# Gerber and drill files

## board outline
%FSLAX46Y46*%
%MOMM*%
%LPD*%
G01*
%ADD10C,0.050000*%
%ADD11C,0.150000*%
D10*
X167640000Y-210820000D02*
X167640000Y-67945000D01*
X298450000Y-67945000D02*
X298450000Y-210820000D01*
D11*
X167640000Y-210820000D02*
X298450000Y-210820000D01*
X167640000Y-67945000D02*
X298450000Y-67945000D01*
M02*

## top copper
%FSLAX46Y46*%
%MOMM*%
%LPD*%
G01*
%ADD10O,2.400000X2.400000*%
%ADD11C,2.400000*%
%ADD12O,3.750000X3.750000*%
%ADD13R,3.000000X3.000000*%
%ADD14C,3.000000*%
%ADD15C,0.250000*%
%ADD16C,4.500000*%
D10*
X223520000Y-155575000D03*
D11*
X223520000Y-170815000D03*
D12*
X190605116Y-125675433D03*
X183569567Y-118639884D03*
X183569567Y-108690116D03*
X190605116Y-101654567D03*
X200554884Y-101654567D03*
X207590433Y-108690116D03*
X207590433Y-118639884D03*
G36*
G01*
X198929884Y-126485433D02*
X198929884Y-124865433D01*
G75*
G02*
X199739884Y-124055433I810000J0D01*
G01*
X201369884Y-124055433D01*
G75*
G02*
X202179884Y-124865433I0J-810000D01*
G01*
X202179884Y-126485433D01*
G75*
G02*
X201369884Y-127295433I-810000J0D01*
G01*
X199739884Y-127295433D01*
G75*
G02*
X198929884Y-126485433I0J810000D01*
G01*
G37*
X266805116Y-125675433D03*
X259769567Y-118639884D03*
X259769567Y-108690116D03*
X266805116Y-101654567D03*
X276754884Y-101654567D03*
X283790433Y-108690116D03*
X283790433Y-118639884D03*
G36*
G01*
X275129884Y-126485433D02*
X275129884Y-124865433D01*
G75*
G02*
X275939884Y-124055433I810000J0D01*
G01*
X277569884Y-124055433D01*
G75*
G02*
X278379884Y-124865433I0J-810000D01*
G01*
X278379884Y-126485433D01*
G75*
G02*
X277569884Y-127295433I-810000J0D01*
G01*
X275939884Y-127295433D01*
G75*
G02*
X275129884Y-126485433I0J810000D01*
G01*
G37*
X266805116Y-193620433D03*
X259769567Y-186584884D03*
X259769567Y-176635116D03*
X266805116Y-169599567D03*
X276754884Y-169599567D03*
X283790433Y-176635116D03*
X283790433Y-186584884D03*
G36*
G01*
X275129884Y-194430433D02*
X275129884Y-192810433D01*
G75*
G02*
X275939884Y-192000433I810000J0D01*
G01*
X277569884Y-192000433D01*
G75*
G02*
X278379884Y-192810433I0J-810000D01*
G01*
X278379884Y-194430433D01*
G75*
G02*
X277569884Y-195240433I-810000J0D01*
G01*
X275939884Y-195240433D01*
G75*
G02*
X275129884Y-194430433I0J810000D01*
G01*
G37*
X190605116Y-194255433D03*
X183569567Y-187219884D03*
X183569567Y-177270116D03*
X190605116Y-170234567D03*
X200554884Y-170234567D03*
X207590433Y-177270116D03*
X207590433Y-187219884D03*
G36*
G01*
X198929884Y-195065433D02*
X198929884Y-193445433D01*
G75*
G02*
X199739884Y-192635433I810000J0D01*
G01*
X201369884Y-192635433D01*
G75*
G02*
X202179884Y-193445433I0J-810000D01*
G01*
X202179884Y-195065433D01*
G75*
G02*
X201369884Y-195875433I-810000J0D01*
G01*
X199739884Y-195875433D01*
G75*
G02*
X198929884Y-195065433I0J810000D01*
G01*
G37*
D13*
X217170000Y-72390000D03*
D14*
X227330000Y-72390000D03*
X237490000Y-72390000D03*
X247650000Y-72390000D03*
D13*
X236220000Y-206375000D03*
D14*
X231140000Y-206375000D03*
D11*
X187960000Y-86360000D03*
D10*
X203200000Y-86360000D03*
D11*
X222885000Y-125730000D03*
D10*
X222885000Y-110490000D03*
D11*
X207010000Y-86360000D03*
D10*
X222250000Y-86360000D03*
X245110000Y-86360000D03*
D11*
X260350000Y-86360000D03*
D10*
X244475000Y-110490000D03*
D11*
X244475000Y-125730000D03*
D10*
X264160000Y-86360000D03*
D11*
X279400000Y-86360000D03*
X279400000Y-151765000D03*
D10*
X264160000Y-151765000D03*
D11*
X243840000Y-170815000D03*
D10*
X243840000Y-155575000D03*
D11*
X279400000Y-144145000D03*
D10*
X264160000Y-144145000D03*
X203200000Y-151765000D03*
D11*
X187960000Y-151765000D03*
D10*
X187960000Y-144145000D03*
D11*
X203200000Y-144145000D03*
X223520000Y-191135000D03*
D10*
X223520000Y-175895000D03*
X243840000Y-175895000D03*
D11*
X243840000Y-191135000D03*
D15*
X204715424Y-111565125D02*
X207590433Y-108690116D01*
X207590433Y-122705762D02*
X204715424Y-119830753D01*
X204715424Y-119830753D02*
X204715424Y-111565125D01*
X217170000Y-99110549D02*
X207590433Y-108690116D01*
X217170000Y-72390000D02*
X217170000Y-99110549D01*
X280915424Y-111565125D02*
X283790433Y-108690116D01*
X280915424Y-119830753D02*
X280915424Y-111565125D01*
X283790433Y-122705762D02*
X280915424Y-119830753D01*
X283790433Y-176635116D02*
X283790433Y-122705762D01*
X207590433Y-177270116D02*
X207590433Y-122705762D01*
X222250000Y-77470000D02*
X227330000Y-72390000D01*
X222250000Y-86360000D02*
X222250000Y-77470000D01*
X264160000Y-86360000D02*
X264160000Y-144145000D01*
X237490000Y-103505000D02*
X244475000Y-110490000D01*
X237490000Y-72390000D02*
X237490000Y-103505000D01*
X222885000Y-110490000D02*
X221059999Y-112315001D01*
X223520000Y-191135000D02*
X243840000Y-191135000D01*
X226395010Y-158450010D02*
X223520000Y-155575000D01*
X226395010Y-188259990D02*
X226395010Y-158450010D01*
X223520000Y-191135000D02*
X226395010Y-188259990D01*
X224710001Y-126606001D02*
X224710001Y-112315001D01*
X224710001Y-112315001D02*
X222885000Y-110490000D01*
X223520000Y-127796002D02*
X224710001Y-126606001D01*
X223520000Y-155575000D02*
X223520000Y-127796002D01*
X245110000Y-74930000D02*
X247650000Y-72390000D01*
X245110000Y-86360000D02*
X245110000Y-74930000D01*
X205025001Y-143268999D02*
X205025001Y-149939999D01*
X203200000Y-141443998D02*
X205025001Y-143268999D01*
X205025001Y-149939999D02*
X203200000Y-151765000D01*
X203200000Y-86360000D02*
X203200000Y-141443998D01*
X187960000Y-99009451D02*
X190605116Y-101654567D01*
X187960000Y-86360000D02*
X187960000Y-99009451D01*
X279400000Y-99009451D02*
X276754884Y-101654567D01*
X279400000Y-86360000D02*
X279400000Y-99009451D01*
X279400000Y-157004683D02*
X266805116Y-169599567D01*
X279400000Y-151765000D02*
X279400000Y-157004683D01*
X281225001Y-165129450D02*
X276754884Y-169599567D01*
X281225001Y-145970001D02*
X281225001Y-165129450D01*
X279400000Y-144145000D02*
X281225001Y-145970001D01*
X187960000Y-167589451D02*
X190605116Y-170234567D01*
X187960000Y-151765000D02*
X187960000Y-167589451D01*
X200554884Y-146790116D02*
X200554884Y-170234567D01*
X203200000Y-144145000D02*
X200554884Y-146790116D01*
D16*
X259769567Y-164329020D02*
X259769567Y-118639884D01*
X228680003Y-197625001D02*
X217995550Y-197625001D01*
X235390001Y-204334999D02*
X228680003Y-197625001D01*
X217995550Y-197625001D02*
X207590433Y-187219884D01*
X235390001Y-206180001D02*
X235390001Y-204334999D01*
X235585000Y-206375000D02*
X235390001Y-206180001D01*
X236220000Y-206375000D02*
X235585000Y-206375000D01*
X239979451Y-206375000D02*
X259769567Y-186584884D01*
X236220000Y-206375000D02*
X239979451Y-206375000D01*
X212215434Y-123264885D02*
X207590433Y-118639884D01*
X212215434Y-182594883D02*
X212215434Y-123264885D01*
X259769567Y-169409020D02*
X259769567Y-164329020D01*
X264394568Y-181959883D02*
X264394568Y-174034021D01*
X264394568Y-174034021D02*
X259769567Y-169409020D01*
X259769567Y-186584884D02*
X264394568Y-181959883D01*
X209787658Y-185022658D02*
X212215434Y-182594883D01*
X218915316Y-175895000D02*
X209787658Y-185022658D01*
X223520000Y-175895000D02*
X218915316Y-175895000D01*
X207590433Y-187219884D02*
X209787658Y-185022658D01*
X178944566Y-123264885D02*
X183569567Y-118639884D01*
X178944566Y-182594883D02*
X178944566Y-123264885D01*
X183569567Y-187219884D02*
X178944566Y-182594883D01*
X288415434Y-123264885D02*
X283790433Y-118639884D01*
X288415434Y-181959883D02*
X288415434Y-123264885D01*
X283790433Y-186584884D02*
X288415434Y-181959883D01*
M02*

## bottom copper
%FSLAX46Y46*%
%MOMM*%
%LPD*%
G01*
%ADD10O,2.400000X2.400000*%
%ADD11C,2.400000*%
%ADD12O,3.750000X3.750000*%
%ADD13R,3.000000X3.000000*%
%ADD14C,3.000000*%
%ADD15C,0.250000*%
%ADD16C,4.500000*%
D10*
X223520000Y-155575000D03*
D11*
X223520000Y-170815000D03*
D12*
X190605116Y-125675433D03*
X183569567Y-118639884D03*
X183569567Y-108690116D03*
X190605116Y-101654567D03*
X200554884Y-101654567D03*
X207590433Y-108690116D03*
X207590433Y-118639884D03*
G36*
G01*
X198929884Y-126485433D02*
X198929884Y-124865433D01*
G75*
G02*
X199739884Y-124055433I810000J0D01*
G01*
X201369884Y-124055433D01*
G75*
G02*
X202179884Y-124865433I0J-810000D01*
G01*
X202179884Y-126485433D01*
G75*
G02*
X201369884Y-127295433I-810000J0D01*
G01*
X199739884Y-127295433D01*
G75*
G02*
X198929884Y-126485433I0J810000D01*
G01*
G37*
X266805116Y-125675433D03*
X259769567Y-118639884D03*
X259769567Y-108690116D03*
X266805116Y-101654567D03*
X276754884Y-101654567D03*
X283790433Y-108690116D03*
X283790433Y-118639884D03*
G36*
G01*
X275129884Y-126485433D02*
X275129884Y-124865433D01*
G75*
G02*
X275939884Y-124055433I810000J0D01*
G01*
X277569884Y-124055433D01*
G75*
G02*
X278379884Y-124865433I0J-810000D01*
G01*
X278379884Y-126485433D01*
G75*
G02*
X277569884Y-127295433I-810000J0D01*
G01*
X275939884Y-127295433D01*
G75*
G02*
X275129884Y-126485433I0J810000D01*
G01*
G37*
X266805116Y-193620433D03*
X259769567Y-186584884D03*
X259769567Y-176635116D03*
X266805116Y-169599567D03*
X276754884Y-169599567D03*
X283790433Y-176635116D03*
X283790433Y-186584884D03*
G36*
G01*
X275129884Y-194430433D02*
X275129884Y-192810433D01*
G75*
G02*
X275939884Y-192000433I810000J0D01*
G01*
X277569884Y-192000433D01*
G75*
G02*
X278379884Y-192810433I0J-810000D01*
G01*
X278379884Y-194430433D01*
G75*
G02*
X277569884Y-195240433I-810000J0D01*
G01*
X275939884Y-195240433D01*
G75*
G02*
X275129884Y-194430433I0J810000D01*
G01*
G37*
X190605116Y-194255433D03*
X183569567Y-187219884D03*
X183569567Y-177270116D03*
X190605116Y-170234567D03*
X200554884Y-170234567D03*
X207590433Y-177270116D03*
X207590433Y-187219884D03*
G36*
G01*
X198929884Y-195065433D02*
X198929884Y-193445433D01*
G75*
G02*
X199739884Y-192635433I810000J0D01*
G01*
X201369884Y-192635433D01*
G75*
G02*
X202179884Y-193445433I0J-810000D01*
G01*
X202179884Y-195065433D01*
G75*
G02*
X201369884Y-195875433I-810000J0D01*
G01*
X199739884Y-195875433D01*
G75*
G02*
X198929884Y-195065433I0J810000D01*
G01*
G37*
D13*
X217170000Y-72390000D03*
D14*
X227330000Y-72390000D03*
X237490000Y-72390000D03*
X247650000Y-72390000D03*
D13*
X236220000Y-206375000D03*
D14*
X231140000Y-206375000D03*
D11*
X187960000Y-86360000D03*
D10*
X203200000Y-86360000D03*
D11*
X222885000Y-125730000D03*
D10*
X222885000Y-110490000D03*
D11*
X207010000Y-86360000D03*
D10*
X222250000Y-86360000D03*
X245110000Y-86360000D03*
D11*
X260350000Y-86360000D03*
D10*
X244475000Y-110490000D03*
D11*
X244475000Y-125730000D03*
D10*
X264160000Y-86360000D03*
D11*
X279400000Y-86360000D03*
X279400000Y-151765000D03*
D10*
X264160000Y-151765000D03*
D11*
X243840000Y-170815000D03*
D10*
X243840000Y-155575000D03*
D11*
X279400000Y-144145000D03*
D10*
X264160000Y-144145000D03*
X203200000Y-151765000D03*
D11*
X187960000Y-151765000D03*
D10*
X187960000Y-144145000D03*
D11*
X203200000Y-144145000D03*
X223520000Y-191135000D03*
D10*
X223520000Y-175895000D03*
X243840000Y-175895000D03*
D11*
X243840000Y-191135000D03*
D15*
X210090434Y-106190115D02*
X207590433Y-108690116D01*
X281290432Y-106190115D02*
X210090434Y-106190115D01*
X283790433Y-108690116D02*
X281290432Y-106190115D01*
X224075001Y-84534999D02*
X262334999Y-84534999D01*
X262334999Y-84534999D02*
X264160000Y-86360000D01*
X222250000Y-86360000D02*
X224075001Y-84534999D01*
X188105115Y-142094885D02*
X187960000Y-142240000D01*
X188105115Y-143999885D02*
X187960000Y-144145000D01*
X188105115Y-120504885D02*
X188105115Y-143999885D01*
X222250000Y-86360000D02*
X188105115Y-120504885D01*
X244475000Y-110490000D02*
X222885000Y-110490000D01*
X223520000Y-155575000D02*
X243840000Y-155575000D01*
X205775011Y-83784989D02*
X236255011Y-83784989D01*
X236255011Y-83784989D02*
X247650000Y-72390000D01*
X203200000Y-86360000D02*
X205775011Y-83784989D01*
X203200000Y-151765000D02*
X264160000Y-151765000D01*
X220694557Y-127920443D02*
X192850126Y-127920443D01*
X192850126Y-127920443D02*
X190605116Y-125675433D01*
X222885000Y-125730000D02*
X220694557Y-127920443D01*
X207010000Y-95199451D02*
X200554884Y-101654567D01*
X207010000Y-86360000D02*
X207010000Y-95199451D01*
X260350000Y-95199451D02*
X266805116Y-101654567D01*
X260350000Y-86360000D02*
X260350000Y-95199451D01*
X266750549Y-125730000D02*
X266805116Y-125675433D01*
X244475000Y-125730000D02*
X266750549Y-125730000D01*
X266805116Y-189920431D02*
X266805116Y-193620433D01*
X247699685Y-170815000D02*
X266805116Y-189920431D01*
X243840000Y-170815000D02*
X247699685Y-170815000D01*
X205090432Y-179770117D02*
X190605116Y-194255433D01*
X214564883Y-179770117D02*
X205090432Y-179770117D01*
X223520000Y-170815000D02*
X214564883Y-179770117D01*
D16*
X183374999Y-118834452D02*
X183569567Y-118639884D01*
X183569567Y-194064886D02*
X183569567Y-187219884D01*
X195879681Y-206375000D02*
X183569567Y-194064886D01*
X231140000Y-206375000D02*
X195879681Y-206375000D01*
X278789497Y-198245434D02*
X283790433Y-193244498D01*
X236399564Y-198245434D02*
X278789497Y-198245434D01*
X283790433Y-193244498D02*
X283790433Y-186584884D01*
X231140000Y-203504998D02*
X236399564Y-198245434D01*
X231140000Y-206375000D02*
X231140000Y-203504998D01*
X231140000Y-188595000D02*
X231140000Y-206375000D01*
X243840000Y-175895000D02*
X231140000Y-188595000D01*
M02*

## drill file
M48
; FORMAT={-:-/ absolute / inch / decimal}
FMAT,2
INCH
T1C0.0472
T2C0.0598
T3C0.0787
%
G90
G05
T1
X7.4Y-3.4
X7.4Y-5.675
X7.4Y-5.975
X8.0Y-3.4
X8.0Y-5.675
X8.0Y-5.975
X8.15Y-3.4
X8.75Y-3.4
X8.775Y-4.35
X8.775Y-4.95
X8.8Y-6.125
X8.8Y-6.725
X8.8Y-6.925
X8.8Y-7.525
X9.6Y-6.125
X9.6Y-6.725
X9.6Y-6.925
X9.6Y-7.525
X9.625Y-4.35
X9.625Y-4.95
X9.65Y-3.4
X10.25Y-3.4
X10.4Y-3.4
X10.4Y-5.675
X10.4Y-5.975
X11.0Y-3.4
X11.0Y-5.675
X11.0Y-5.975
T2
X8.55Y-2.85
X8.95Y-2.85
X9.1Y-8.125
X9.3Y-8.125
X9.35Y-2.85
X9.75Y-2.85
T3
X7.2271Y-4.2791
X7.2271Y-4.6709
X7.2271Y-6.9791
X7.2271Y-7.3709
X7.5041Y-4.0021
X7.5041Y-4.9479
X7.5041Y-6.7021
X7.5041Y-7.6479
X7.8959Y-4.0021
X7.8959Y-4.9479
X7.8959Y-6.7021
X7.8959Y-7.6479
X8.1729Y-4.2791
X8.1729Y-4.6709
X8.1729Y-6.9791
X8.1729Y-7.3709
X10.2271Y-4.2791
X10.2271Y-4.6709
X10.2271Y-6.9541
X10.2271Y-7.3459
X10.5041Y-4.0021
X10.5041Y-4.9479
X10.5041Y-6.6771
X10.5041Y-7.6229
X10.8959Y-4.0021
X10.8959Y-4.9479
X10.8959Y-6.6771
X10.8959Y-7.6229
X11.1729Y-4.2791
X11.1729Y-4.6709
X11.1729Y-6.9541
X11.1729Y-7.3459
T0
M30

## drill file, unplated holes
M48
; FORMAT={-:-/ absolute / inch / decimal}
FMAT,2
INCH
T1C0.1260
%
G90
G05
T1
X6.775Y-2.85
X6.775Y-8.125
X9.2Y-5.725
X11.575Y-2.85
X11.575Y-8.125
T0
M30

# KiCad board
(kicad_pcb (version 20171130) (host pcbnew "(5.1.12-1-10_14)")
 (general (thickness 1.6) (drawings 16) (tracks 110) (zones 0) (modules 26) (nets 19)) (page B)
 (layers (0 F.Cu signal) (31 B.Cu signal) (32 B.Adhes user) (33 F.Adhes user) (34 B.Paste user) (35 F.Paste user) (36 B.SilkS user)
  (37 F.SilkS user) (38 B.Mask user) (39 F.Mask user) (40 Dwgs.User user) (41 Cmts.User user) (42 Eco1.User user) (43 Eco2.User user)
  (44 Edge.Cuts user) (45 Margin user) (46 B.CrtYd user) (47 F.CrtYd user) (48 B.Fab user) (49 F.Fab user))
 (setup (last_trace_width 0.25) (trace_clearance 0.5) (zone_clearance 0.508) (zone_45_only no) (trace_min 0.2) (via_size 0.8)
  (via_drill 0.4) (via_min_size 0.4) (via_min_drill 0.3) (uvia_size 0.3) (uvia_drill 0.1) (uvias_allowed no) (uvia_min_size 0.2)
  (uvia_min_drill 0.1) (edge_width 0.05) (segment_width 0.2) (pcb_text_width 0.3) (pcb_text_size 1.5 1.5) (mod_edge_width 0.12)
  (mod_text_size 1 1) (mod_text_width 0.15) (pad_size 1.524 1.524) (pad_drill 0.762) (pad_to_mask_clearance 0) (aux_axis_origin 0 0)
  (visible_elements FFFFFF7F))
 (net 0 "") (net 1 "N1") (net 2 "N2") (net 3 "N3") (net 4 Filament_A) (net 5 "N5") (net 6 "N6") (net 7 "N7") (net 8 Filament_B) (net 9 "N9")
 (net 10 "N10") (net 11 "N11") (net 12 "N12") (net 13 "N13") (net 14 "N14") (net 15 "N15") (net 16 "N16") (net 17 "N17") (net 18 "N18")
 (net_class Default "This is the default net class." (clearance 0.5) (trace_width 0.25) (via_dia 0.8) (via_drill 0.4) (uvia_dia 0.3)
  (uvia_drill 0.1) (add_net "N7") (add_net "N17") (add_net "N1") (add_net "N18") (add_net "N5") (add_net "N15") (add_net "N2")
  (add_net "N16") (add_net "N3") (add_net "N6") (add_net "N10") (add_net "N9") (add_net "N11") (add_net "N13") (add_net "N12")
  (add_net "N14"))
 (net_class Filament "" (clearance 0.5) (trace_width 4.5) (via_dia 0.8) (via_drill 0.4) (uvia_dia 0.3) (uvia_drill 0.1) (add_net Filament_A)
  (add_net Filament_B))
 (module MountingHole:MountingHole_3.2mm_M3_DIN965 (layer F.Cu) (at 294.005 206.375)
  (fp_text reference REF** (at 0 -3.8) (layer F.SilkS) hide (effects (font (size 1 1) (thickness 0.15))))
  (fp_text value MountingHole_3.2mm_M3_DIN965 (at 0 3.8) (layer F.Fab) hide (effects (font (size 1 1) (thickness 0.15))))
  (pad 1 np_thru_hole circle (at 0 0) (size 3.2 3.2) (drill 3.2) (layers *.Cu *.Mask)))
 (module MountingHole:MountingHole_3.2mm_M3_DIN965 (layer F.Cu) (at 172.085 206.375)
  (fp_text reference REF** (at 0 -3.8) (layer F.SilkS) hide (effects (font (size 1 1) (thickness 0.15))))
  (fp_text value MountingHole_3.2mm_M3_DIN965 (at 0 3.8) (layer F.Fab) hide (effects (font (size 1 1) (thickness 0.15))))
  (pad 1 np_thru_hole circle (at 0 0) (size 3.2 3.2) (drill 3.2) (layers *.Cu *.Mask)))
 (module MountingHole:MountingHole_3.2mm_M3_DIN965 (layer F.Cu) (at 172.085 72.39)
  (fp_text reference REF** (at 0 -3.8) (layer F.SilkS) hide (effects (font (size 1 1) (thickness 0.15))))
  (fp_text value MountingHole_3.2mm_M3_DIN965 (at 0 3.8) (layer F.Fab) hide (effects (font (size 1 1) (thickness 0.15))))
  (pad 1 np_thru_hole circle (at 0 0) (size 3.2 3.2) (drill 3.2) (layers *.Cu *.Mask)))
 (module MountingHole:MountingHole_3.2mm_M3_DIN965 (layer F.Cu) (at 294.005 72.39)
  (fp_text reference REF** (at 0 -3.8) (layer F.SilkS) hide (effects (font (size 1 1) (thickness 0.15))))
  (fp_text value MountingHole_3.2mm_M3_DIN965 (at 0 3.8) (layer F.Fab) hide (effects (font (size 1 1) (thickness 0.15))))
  (pad 1 np_thru_hole circle (at 0 0) (size 3.2 3.2) (drill 3.2) (layers *.Cu *.Mask)))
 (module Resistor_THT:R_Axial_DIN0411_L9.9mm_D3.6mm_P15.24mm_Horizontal (layer F.Cu) (at 223.52 170.815 90)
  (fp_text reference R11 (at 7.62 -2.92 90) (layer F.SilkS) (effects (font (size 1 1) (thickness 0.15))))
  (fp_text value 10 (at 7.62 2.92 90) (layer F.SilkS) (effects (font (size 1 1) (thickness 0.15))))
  (pad 2 thru_hole oval (at 15.24 0 90) (size 2.4 2.4) (drill 1.2) (layers *.Cu *.Mask) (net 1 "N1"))
  (pad 1 thru_hole circle (at 0 0 90) (size 2.4 2.4) (drill 1.2) (layers *.Cu *.Mask) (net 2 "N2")))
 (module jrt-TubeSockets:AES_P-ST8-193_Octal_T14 (layer F.Cu) (at 195.58 113.665)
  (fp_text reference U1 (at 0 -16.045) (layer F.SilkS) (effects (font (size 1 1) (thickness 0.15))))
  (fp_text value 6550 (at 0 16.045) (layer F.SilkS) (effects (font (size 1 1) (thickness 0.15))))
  (pad 8 thru_hole oval (at -4.974884 12.010433) (size 3.75 3.75) (drill 2) (layers *.Cu *.Mask) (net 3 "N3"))
  (pad 7 thru_hole oval (at -12.010433 4.974884) (size 3.75 3.75) (drill 2) (layers *.Cu *.Mask) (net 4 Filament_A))
  (pad 6 thru_hole oval (at -12.010433 -4.974884) (size 3.75 3.75) (drill 2) (layers *.Cu *.Mask))
  (pad 5 thru_hole oval (at -4.974884 -12.010433) (size 3.75 3.75) (drill 2) (layers *.Cu *.Mask) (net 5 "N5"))
  (pad 4 thru_hole oval (at 4.974884 -12.010433) (size 3.75 3.75) (drill 2) (layers *.Cu *.Mask) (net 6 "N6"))
  (pad 3 thru_hole oval (at 12.010433 -4.974884) (size 3.75 3.75) (drill 2) (layers *.Cu *.Mask) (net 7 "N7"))
  (pad 2 thru_hole oval (at 12.010433 4.974884) (size 3.75 3.75) (drill 2) (layers *.Cu *.Mask) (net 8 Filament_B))
  (pad 1 thru_hole roundrect (at 4.974884 12.010433) (size 3.25 3.24) (drill 2) (layers *.Cu *.Mask) (roundrect_rratio 0.25)))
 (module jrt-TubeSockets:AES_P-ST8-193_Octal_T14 (layer F.Cu) (at 271.78 113.665)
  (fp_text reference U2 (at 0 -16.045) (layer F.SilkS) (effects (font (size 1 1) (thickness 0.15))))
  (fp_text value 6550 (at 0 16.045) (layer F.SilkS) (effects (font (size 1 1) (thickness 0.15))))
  (pad 8 thru_hole oval (at -4.974884 12.010433) (size 3.75 3.75) (drill 2) (layers *.Cu *.Mask) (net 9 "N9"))
  (pad 7 thru_hole oval (at -12.010433 4.974884) (size 3.75 3.75) (drill 2) (layers *.Cu *.Mask) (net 8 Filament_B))
  (pad 6 thru_hole oval (at -12.010433 -4.974884) (size 3.75 3.75) (drill 2) (layers *.Cu *.Mask))
  (pad 5 thru_hole oval (at -4.974884 -12.010433) (size 3.75 3.75) (drill 2) (layers *.Cu *.Mask) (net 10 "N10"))
  (pad 4 thru_hole oval (at 4.974884 -12.010433) (size 3.75 3.75) (drill 2) (layers *.Cu *.Mask) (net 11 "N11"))
  (pad 3 thru_hole oval (at 12.010433 -4.974884) (size 3.75 3.75) (drill 2) (layers *.Cu *.Mask) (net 7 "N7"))
  (pad 2 thru_hole oval (at 12.010433 4.974884) (size 3.75 3.75) (drill 2) (layers *.Cu *.Mask) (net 4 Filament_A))
  (pad 1 thru_hole roundrect (at 4.974884 12.010433) (size 3.25 3.24) (drill 2) (layers *.Cu *.Mask) (roundrect_rratio 0.25)))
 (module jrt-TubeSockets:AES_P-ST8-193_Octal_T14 (layer F.Cu) (at 271.78 181.61)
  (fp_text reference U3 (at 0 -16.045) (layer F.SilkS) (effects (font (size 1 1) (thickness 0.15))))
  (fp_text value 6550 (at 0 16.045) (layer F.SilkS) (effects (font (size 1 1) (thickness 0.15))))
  (pad 8 thru_hole oval (at -4.974884 12.010433) (size 3.75 3.75) (drill 2) (layers *.Cu *.Mask) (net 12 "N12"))
  (pad 7 thru_hole oval (at -12.010433 4.974884) (size 3.75 3.75) (drill 2) (layers *.Cu *.Mask) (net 8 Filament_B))
  (pad 6 thru_hole oval (at -12.010433 -4.974884) (size 3.75 3.75) (drill 2) (layers *.Cu *.Mask))
  (pad 5 thru_hole oval (at -4.974884 -12.010433) (size 3.75 3.75) (drill 2) (layers *.Cu *.Mask) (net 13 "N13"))
  (pad 4 thru_hole oval (at 4.974884 -12.010433) (size 3.75 3.75) (drill 2) (layers *.Cu *.Mask) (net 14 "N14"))
  (pad 3 thru_hole oval (at 12.010433 -4.974884) (size 3.75 3.75) (drill 2) (layers *.Cu *.Mask) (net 7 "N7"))
  (pad 2 thru_hole oval (at 12.010433 4.974884) (size 3.75 3.75) (drill 2) (layers *.Cu *.Mask) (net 4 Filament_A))
  (pad 1 thru_hole roundrect (at 4.974884 12.010433) (size 3.25 3.24) (drill 2) (layers *.Cu *.Mask) (roundrect_rratio 0.25)))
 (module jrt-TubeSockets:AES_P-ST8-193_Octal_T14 (layer F.Cu) (at 195.58 182.245)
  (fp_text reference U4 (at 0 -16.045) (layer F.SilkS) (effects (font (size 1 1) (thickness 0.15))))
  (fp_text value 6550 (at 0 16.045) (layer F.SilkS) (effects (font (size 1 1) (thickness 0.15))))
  (pad 8 thru_hole oval (at -4.974884 12.010433) (size 3.75 3.75) (drill 2) (layers *.Cu *.Mask) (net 2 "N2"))
  (pad 7 thru_hole oval (at -12.010433 4.974884) (size 3.75 3.75) (drill 2) (layers *.Cu *.Mask) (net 4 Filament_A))
  (pad 6 thru_hole oval (at -12.010433 -4.974884) (size 3.75 3.75) (drill 2) (layers *.Cu *.Mask))
  (pad 5 thru_hole oval (at -4.974884 -12.010433) (size 3.75 3.75) (drill 2) (layers *.Cu *.Mask) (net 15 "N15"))
  (pad 4 thru_hole oval (at 4.974884 -12.010433) (size 3.75 3.75) (drill 2) (layers *.Cu *.Mask) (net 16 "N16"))
  (pad 3 thru_hole oval (at 12.010433 -4.974884) (size 3.75 3.75) (drill 2) (layers *.Cu *.Mask) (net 7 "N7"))
  (pad 2 thru_hole oval (at 12.010433 4.974884) (size 3.75 3.75) (drill 2) (layers *.Cu *.Mask) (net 8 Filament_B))
  (pad 1 thru_hole roundrect (at 4.974884 12.010433) (size 3.25 3.24) (drill 2) (layers *.Cu *.Mask) (roundrect_rratio 0.25)))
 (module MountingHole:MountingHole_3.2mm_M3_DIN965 (layer F.Cu) (at 233.68 145.415)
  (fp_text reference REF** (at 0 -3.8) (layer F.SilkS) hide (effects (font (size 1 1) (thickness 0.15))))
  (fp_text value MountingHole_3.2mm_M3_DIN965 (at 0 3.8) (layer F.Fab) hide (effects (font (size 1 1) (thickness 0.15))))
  (pad 1 np_thru_hole circle (at 0 0) (size 3.2 3.2) (drill 3.2) (layers *.Cu *.Mask)))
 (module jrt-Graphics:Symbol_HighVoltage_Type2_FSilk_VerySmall (layer F.Cu) (at 233.68 123.825)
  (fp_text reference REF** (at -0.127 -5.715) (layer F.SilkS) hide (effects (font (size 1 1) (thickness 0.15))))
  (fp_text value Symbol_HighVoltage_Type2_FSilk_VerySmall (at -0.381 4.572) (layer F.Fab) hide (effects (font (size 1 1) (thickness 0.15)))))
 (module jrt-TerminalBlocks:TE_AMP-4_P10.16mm (layer F.Cu) (at 232.41 72.39)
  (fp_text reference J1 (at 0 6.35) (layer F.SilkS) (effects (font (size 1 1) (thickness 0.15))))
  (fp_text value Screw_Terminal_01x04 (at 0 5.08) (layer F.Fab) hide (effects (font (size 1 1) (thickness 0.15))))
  (pad 1 thru_hole rect (at -15.24 0) (size 3 3) (drill 1.52) (layers *.Cu *.Mask) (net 7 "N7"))
  (pad 2 thru_hole circle (at -5.08 0) (size 3 3) (drill 1.52) (layers *.Cu *.Mask) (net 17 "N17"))
  (pad 3 thru_hole circle (at 5.08 0) (size 3 3) (drill 1.52) (layers *.Cu *.Mask) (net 1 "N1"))
  (pad 4 thru_hole circle (at 15.24 0) (size 3 3) (drill 1.52) (layers *.Cu *.Mask) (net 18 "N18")))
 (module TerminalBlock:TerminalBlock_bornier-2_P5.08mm (layer F.Cu) (at 236.22 206.375 180)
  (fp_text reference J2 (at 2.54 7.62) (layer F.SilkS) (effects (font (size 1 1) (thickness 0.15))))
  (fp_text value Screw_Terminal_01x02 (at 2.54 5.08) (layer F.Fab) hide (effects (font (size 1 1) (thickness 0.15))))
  (pad 1 thru_hole rect (at 0 0 180) (size 3 3) (drill 1.52) (layers *.Cu *.Mask) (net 8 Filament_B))
  (pad 2 thru_hole circle (at 5.08 0 180) (size 3 3) (drill 1.52) (layers *.Cu *.Mask) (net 4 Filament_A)))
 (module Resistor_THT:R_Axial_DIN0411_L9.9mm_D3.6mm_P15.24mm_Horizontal (layer F.Cu) (at 187.96 86.36)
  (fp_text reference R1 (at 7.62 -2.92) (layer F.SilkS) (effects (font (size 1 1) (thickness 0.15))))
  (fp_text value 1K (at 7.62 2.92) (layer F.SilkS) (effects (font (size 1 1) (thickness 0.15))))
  (pad 1 thru_hole circle (at 0 0) (size 2.4 2.4) (drill 1.2) (layers *.Cu *.Mask) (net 5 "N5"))
  (pad 2 thru_hole oval (at 15.24 0) (size 2.4 2.4) (drill 1.2) (layers *.Cu *.Mask) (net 18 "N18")))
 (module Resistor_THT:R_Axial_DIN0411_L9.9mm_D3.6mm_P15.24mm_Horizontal (layer F.Cu) (at 222.885 125.73 90)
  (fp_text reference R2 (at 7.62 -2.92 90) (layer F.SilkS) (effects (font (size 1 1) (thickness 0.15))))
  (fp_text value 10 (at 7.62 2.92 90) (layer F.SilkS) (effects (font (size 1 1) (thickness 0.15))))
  (pad 1 thru_hole circle (at 0 0 90) (size 2.4 2.4) (drill 1.2) (layers *.Cu *.Mask) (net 3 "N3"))
  (pad 2 thru_hole oval (at 15.24 0 90) (size 2.4 2.4) (drill 1.2) (layers *.Cu *.Mask) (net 1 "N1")))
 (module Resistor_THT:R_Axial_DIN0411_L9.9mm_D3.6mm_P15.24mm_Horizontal (layer F.Cu) (at 207.01 86.36)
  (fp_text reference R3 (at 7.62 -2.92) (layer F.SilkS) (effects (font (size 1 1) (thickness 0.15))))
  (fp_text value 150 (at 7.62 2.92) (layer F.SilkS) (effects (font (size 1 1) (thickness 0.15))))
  (pad 1 thru_hole circle (at 0 0) (size 2.4 2.4) (drill 1.2) (layers *.Cu *.Mask) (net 6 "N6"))
  (pad 2 thru_hole oval (at 15.24 0) (size 2.4 2.4) (drill 1.2) (layers *.Cu *.Mask) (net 17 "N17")))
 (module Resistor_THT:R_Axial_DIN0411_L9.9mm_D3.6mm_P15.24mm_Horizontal (layer F.Cu) (at 260.35 86.36 180)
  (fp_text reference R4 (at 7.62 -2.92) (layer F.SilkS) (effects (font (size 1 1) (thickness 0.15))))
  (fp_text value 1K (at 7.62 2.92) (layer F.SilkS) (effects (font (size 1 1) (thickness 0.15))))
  (pad 2 thru_hole oval (at 15.24 0 180) (size 2.4 2.4) (drill 1.2) (layers *.Cu *.Mask) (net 18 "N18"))
  (pad 1 thru_hole circle (at 0 0 180) (size 2.4 2.4) (drill 1.2) (layers *.Cu *.Mask) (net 10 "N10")))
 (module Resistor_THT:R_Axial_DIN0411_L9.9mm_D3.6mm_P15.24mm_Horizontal (layer F.Cu) (at 244.475 125.73 90)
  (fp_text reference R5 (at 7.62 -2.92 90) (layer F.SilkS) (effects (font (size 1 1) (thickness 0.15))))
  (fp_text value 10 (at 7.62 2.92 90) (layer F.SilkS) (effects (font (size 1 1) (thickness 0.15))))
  (pad 2 thru_hole oval (at 15.24 0 90) (size 2.4 2.4) (drill 1.2) (layers *.Cu *.Mask) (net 1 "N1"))
  (pad 1 thru_hole circle (at 0 0 90) (size 2.4 2.4) (drill 1.2) (layers *.Cu *.Mask) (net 9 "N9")))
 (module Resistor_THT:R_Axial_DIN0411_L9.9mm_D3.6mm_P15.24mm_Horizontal (layer F.Cu) (at 279.4 86.36 180)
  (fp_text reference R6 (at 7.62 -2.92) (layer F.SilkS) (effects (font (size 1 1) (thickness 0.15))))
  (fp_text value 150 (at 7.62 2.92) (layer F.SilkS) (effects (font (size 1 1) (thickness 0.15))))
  (pad 2 thru_hole oval (at 15.24 0 180) (size 2.4 2.4) (drill 1.2) (layers *.Cu *.Mask) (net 17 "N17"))
  (pad 1 thru_hole circle (at 0 0 180) (size 2.4 2.4) (drill 1.2) (layers *.Cu *.Mask) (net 11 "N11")))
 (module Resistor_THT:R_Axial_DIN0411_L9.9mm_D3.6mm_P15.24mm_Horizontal (layer F.Cu) (at 279.4 151.765 180)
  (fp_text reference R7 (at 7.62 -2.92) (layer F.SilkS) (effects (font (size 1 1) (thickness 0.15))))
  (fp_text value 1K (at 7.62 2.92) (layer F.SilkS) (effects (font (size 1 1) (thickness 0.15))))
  (pad 1 thru_hole circle (at 0 0 180) (size 2.4 2.4) (drill 1.2) (layers *.Cu *.Mask) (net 13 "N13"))
  (pad 2 thru_hole oval (at 15.24 0 180) (size 2.4 2.4) (drill 1.2) (layers *.Cu *.Mask) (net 18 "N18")))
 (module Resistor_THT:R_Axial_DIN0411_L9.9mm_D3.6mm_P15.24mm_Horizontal (layer F.Cu) (at 243.84 170.815 90)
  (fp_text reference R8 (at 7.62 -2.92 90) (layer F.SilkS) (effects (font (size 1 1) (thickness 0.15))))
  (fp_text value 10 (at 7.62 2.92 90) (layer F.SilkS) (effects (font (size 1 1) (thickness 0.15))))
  (pad 1 thru_hole circle (at 0 0 90) (size 2.4 2.4) (drill 1.2) (layers *.Cu *.Mask) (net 12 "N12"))
  (pad 2 thru_hole oval (at 15.24 0 90) (size 2.4 2.4) (drill 1.2) (layers *.Cu *.Mask) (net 1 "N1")))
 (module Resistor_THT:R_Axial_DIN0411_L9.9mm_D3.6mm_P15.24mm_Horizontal (layer F.Cu) (at 279.4 144.145 180)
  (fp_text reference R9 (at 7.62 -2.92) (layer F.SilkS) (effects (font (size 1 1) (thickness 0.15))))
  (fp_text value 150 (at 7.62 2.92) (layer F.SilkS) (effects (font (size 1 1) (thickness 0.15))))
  (pad 1 thru_hole circle (at 0 0 180) (size 2.4 2.4) (drill 1.2) (layers *.Cu *.Mask) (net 14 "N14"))
  (pad 2 thru_hole oval (at 15.24 0 180) (size 2.4 2.4) (drill 1.2) (layers *.Cu *.Mask) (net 17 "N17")))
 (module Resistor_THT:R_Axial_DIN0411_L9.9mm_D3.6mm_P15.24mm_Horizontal (layer F.Cu) (at 187.96 151.765)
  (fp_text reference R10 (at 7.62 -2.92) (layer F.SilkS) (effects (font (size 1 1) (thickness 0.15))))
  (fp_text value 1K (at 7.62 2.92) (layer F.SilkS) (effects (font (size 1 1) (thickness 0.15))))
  (pad 2 thru_hole oval (at 15.24 0) (size 2.4 2.4) (drill 1.2) (layers *.Cu *.Mask) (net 18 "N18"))
  (pad 1 thru_hole circle (at 0 0) (size 2.4 2.4) (drill 1.2) (layers *.Cu *.Mask) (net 15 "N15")))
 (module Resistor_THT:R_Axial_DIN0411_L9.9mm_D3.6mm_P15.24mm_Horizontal (layer F.Cu) (at 203.2 144.145 180)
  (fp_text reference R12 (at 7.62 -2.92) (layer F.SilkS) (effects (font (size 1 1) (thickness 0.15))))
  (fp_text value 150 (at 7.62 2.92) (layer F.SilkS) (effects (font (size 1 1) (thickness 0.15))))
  (pad 2 thru_hole oval (at 15.24 0 180) (size 2.4 2.4) (drill 1.2) (layers *.Cu *.Mask) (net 17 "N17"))
  (pad 1 thru_hole circle (at 0 0 180) (size 2.4 2.4) (drill 1.2) (layers *.Cu *.Mask) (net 16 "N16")))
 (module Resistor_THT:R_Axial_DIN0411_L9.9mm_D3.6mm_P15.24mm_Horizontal (layer F.Cu) (at 223.52 191.135 90)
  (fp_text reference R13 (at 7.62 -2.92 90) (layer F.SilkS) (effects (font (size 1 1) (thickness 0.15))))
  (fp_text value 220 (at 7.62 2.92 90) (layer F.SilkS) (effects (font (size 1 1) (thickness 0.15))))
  (pad 1 thru_hole circle (at 0 0 90) (size 2.4 2.4) (drill 1.2) (layers *.Cu *.Mask) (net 1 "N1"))
  (pad 2 thru_hole oval (at 15.24 0 90) (size 2.4 2.4) (drill 1.2) (layers *.Cu *.Mask) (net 8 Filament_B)))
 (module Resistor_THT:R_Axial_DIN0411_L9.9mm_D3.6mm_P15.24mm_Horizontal (layer F.Cu) (at 243.84 191.135 90)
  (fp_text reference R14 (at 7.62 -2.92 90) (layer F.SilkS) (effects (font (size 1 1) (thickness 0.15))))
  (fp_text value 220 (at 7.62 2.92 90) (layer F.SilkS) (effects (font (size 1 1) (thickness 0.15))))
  (pad 2 thru_hole oval (at 15.24 0 90) (size 2.4 2.4) (drill 1.2) (layers *.Cu *.Mask) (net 4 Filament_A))
  (pad 1 thru_hole circle (at 0 0 90) (size 2.4 2.4) (drill 1.2) (layers *.Cu *.Mask) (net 1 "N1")))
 (gr_line (start 167.64 210.82) (end 167.64 67.945) (layer Edge.Cuts) (width 0.05))
 (gr_line (start 298.45 67.945) (end 298.45 210.82) (layer Edge.Cuts) (width 0.05))
 (gr_line (start 167.64 210.82) (end 298.45 210.82) (layer Edge.Cuts) (width 0.15))
 (gr_line (start 167.64 67.945) (end 298.45 67.945) (layer Edge.Cuts) (width 0.15))
 (segment (start 204.715424 111.565125) (end 207.590433 108.690116) (width 0.25) (layer F.Cu) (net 7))
 (segment (start 207.590433 122.705762) (end 204.715424 119.830753) (width 0.25) (layer F.Cu) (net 7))
 (segment (start 204.715424 119.830753) (end 204.715424 111.565125) (width 0.25) (layer F.Cu) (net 7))
 (segment (start 217.17 99.110549) (end 207.590433 108.690116) (width 0.25) (layer F.Cu) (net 7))
 (segment (start 217.17 72.39) (end 217.17 99.110549) (width 0.25) (layer F.Cu) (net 7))
 (segment (start 210.090434 106.190115) (end 207.590433 108.690116) (width 0.25) (layer B.Cu) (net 7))
 (segment (start 281.290432 106.190115) (end 210.090434 106.190115) (width 0.25) (layer B.Cu) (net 7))
 (segment (start 283.790433 108.690116) (end 281.290432 106.190115) (width 0.25) (layer B.Cu) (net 7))
 (segment (start 280.915424 111.565125) (end 283.790433 108.690116) (width 0.25) (layer F.Cu) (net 7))
 (segment (start 280.915424 119.830753) (end 280.915424 111.565125) (width 0.25) (layer F.Cu) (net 7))
 (segment (start 283.790433 122.705762) (end 280.915424 119.830753) (width 0.25) (layer F.Cu) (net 7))
 (segment (start 283.790433 176.635116) (end 283.790433 122.705762) (width 0.25) (layer F.Cu) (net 7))
 (segment (start 207.590433 177.270116) (end 207.590433 122.705762) (width 0.25) (layer F.Cu) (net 7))
 (segment (start 224.075001 84.534999) (end 262.334999 84.534999) (width 0.25) (layer B.Cu) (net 17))
 (segment (start 262.334999 84.534999) (end 264.16 86.36) (width 0.25) (layer B.Cu) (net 17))
 (segment (start 222.25 86.36) (end 224.075001 84.534999) (width 0.25) (layer B.Cu) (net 17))
 (segment (start 222.25 77.47) (end 227.33 72.39) (width 0.25) (layer F.Cu) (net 17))
 (segment (start 222.25 86.36) (end 222.25 77.47) (width 0.25) (layer F.Cu) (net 17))
 (segment (start 188.105115 142.094885) (end 187.96 142.24) (width 0.25) (layer B.Cu) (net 17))
 (segment (start 188.105115 143.999885) (end 187.96 144.145) (width 0.25) (layer B.Cu) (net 17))
 (segment (start 188.105115 120.504885) (end 188.105115 143.999885) (width 0.25) (layer B.Cu) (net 17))
 (segment (start 222.25 86.36) (end 188.105115 120.504885) (width 0.25) (layer B.Cu) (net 17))
 (segment (start 264.16 86.36) (end 264.16 144.145) (width 0.25) (layer F.Cu) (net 17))
 (segment (start 237.49 103.505) (end 244.475 110.49) (width 0.25) (layer F.Cu) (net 1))
 (segment (start 237.49 72.39) (end 237.49 103.505) (width 0.25) (layer F.Cu) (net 1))
 (segment (start 244.475 110.49) (end 222.885 110.49) (width 0.25) (layer B.Cu) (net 1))
 (segment (start 222.885 110.49) (end 221.059999 112.315001) (width 0.25) (layer F.Cu) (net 1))
 (segment (start 223.52 155.575) (end 243.84 155.575) (width 0.25) (layer B.Cu) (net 1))
 (segment (start 223.52 191.135) (end 243.84 191.135) (width 0.25) (layer F.Cu) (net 1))
 (segment (start 226.39501 158.45001) (end 223.52 155.575) (width 0.25) (layer F.Cu) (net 1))
 (segment (start 226.39501 188.25999) (end 226.39501 158.45001) (width 0.25) (layer F.Cu) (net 1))
 (segment (start 223.52 191.135) (end 226.39501 188.25999) (width 0.25) (layer F.Cu) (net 1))
 (segment (start 224.710001 126.606001) (end 224.710001 112.315001) (width 0.25) (layer F.Cu) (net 1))
 (segment (start 224.710001 112.315001) (end 222.885 110.49) (width 0.25) (layer F.Cu) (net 1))
 (segment (start 223.52 127.796002) (end 224.710001 126.606001) (width 0.25) (layer F.Cu) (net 1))
 (segment (start 223.52 155.575) (end 223.52 127.796002) (width 0.25) (layer F.Cu) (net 1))
 (segment (start 245.11 74.93) (end 247.65 72.39) (width 0.25) (layer F.Cu) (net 18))
 (segment (start 245.11 86.36) (end 245.11 74.93) (width 0.25) (layer F.Cu) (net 18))
 (segment (start 205.775011 83.784989) (end 236.255011 83.784989) (width 0.25) (layer B.Cu) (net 18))
 (segment (start 236.255011 83.784989) (end 247.65 72.39) (width 0.25) (layer B.Cu) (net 18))
 (segment (start 203.2 86.36) (end 205.775011 83.784989) (width 0.25) (layer B.Cu) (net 18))
 (segment (start 203.2 151.765) (end 264.16 151.765) (width 0.25) (layer B.Cu) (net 18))
 (segment (start 205.025001 143.268999) (end 205.025001 149.939999) (width 0.25) (layer F.Cu) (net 18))
 (segment (start 203.2 141.443998) (end 205.025001 143.268999) (width 0.25) (layer F.Cu) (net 18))
 (segment (start 205.025001 149.939999) (end 203.2 151.765) (width 0.25) (layer F.Cu) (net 18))
 (segment (start 203.2 86.36) (end 203.2 141.443998) (width 0.25) (layer F.Cu) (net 18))
 (segment (start 187.96 99.009451) (end 190.605116 101.654567) (width 0.25) (layer F.Cu) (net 5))
 (segment (start 187.96 86.36) (end 187.96 99.009451) (width 0.25) (layer F.Cu) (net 5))
 (segment (start 220.694557 127.920443) (end 192.850126 127.920443) (width 0.25) (layer B.Cu) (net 3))
 (segment (start 192.850126 127.920443) (end 190.605116 125.675433) (width 0.25) (layer B.Cu) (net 3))
 (segment (start 222.885 125.73) (end 220.694557 127.920443) (width 0.25) (layer B.Cu) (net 3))
 (segment (start 207.01 95.199451) (end 200.554884 101.654567) (width 0.25) (layer B.Cu) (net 6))
 (segment (start 207.01 86.36) (end 207.01 95.199451) (width 0.25) (layer B.Cu) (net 6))
 (segment (start 260.35 95.199451) (end 266.805116 101.654567) (width 0.25) (layer B.Cu) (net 10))
 (segment (start 260.35 86.36) (end 260.35 95.199451) (width 0.25) (layer B.Cu) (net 10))
 (segment (start 266.750549 125.73) (end 266.805116 125.675433) (width 0.25) (layer B.Cu) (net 9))
 (segment (start 244.475 125.73) (end 266.750549 125.73) (width 0.25) (layer B.Cu) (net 9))
 (segment (start 279.4 99.009451) (end 276.754884 101.654567) (width 0.25) (layer F.Cu) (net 11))
 (segment (start 279.4 86.36) (end 279.4 99.009451) (width 0.25) (layer F.Cu) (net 11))
 (segment (start 279.4 157.004683) (end 266.805116 169.599567) (width 0.25) (layer F.Cu) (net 13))
 (segment (start 279.4 151.765) (end 279.4 157.004683) (width 0.25) (layer F.Cu) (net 13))
 (segment (start 266.805116 189.920431) (end 266.805116 193.620433) (width 0.25) (layer B.Cu) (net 12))
 (segment (start 247.699685 170.815) (end 266.805116 189.920431) (width 0.25) (layer B.Cu) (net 12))
 (segment (start 243.84 170.815) (end 247.699685 170.815) (width 0.25) (layer B.Cu) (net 12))
 (segment (start 281.225001 165.12945) (end 276.754884 169.599567) (width 0.25) (layer F.Cu) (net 14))
 (segment (start 281.225001 145.970001) (end 281.225001 165.12945) (width 0.25) (layer F.Cu) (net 14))
 (segment (start 279.4 144.145) (end 281.225001 145.970001) (width 0.25) (layer F.Cu) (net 14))
 (segment (start 187.96 167.589451) (end 190.605116 170.234567) (width 0.25) (layer F.Cu) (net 15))
 (segment (start 187.96 151.765) (end 187.96 167.589451) (width 0.25) (layer F.Cu) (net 15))
 (segment (start 205.090432 179.770117) (end 190.605116 194.255433) (width 0.25) (layer B.Cu) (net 2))
 (segment (start 214.564883 179.770117) (end 205.090432 179.770117) (width 0.25) (layer B.Cu) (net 2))
 (segment (start 223.52 170.815) (end 214.564883 179.770117) (width 0.25) (layer B.Cu) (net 2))
 (segment (start 200.554884 146.790116) (end 200.554884 170.234567) (width 0.25) (layer F.Cu) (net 16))
 (segment (start 203.2 144.145) (end 200.554884 146.790116) (width 0.25) (layer F.Cu) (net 16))
 (segment (start 259.769567 164.32902) (end 259.769567 118.639884) (width 4.5) (layer F.Cu) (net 8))
 (segment (start 228.680003 197.625001) (end 217.99555 197.625001) (width 4.5) (layer F.Cu) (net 8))
 (segment (start 235.390001 204.334999) (end 228.680003 197.625001) (width 4.5) (layer F.Cu) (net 8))
 (segment (start 217.99555 197.625001) (end 207.590433 187.219884) (width 4.5) (layer F.Cu) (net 8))
 (segment (start 235.390001 206.180001) (end 235.390001 204.334999) (width 4.5) (layer F.Cu) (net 8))
 (segment (start 235.585 206.375) (end 235.390001 206.180001) (width 4.5) (layer F.Cu) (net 8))
 (segment (start 236.22 206.375) (end 235.585 206.375) (width 4.5) (layer F.Cu) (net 8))
 (segment (start 239.979451 206.375) (end 259.769567 186.584884) (width 4.5) (layer F.Cu) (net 8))
 (segment (start 236.22 206.375) (end 239.979451 206.375) (width 4.5) (layer F.Cu) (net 8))
 (segment (start 212.215434 123.264885) (end 207.590433 118.639884) (width 4.5) (layer F.Cu) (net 8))
 (segment (start 212.215434 182.594883) (end 212.215434 123.264885) (width 4.5) (layer F.Cu) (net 8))
 (segment (start 259.769567 169.40902) (end 259.769567 164.32902) (width 4.5) (layer F.Cu) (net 8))
 (segment (start 264.394568 181.959883) (end 264.394568 174.034021) (width 4.5) (layer F.Cu) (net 8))
 (segment (start 264.394568 174.034021) (end 259.769567 169.40902) (width 4.5) (layer F.Cu) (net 8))
 (segment (start 259.769567 186.584884) (end 264.394568 181.959883) (width 4.5) (layer F.Cu) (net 8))
 (segment (start 209.787658 185.022658) (end 212.215434 182.594883) (width 4.5) (layer F.Cu) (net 8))
 (segment (start 218.915316 175.895) (end 209.787658 185.022658) (width 4.5) (layer F.Cu) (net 8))
 (segment (start 223.52 175.895) (end 218.915316 175.895) (width 4.5) (layer F.Cu) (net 8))
 (segment (start 207.590433 187.219884) (end 209.787658 185.022658) (width 4.5) (layer F.Cu) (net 8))
 (segment (start 183.374999 118.834452) (end 183.569567 118.639884) (width 4.5) (layer B.Cu) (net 4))
 (segment (start 183.569567 194.064886) (end 183.569567 187.219884) (width 4.5) (layer B.Cu) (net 4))
 (segment (start 195.879681 206.375) (end 183.569567 194.064886) (width 4.5) (layer B.Cu) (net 4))
 (segment (start 231.14 206.375) (end 195.879681 206.375) (width 4.5) (layer B.Cu) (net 4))
 (segment (start 278.789497 198.245434) (end 283.790433 193.244498) (width 4.5) (layer B.Cu) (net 4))
 (segment (start 236.399564 198.245434) (end 278.789497 198.245434) (width 4.5) (layer B.Cu) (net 4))
 (segment (start 283.790433 193.244498) (end 283.790433 186.584884) (width 4.5) (layer B.Cu) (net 4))
 (segment (start 231.14 203.504998) (end 236.399564 198.245434) (width 4.5) (layer B.Cu) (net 4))
 (segment (start 231.14 206.375) (end 231.14 203.504998) (width 4.5) (layer B.Cu) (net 4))
 (segment (start 231.14 188.595) (end 231.14 206.375) (width 4.5) (layer B.Cu) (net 4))
 (segment (start 243.84 175.895) (end 231.14 188.595) (width 4.5) (layer B.Cu) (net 4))
 (segment (start 178.944566 123.264885) (end 183.569567 118.639884) (width 4.5) (layer F.Cu) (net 4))
 (segment (start 178.944566 182.594883) (end 178.944566 123.264885) (width 4.5) (layer F.Cu) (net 4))
 (segment (start 183.569567 187.219884) (end 178.944566 182.594883) (width 4.5) (layer F.Cu) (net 4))
 (segment (start 288.415434 123.264885) (end 283.790433 118.639884) (width 4.5) (layer F.Cu) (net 4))
 (segment (start 288.415434 181.959883) (end 288.415434 123.264885) (width 4.5) (layer F.Cu) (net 4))
 (segment (start 283.790433 186.584884) (end 288.415434 181.959883) (width 4.5) (layer F.Cu) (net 4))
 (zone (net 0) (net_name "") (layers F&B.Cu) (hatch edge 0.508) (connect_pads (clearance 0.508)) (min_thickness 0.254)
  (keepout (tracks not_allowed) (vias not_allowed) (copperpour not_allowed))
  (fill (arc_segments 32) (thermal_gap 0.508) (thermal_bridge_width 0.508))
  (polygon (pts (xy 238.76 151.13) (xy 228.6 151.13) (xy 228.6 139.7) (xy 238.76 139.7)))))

